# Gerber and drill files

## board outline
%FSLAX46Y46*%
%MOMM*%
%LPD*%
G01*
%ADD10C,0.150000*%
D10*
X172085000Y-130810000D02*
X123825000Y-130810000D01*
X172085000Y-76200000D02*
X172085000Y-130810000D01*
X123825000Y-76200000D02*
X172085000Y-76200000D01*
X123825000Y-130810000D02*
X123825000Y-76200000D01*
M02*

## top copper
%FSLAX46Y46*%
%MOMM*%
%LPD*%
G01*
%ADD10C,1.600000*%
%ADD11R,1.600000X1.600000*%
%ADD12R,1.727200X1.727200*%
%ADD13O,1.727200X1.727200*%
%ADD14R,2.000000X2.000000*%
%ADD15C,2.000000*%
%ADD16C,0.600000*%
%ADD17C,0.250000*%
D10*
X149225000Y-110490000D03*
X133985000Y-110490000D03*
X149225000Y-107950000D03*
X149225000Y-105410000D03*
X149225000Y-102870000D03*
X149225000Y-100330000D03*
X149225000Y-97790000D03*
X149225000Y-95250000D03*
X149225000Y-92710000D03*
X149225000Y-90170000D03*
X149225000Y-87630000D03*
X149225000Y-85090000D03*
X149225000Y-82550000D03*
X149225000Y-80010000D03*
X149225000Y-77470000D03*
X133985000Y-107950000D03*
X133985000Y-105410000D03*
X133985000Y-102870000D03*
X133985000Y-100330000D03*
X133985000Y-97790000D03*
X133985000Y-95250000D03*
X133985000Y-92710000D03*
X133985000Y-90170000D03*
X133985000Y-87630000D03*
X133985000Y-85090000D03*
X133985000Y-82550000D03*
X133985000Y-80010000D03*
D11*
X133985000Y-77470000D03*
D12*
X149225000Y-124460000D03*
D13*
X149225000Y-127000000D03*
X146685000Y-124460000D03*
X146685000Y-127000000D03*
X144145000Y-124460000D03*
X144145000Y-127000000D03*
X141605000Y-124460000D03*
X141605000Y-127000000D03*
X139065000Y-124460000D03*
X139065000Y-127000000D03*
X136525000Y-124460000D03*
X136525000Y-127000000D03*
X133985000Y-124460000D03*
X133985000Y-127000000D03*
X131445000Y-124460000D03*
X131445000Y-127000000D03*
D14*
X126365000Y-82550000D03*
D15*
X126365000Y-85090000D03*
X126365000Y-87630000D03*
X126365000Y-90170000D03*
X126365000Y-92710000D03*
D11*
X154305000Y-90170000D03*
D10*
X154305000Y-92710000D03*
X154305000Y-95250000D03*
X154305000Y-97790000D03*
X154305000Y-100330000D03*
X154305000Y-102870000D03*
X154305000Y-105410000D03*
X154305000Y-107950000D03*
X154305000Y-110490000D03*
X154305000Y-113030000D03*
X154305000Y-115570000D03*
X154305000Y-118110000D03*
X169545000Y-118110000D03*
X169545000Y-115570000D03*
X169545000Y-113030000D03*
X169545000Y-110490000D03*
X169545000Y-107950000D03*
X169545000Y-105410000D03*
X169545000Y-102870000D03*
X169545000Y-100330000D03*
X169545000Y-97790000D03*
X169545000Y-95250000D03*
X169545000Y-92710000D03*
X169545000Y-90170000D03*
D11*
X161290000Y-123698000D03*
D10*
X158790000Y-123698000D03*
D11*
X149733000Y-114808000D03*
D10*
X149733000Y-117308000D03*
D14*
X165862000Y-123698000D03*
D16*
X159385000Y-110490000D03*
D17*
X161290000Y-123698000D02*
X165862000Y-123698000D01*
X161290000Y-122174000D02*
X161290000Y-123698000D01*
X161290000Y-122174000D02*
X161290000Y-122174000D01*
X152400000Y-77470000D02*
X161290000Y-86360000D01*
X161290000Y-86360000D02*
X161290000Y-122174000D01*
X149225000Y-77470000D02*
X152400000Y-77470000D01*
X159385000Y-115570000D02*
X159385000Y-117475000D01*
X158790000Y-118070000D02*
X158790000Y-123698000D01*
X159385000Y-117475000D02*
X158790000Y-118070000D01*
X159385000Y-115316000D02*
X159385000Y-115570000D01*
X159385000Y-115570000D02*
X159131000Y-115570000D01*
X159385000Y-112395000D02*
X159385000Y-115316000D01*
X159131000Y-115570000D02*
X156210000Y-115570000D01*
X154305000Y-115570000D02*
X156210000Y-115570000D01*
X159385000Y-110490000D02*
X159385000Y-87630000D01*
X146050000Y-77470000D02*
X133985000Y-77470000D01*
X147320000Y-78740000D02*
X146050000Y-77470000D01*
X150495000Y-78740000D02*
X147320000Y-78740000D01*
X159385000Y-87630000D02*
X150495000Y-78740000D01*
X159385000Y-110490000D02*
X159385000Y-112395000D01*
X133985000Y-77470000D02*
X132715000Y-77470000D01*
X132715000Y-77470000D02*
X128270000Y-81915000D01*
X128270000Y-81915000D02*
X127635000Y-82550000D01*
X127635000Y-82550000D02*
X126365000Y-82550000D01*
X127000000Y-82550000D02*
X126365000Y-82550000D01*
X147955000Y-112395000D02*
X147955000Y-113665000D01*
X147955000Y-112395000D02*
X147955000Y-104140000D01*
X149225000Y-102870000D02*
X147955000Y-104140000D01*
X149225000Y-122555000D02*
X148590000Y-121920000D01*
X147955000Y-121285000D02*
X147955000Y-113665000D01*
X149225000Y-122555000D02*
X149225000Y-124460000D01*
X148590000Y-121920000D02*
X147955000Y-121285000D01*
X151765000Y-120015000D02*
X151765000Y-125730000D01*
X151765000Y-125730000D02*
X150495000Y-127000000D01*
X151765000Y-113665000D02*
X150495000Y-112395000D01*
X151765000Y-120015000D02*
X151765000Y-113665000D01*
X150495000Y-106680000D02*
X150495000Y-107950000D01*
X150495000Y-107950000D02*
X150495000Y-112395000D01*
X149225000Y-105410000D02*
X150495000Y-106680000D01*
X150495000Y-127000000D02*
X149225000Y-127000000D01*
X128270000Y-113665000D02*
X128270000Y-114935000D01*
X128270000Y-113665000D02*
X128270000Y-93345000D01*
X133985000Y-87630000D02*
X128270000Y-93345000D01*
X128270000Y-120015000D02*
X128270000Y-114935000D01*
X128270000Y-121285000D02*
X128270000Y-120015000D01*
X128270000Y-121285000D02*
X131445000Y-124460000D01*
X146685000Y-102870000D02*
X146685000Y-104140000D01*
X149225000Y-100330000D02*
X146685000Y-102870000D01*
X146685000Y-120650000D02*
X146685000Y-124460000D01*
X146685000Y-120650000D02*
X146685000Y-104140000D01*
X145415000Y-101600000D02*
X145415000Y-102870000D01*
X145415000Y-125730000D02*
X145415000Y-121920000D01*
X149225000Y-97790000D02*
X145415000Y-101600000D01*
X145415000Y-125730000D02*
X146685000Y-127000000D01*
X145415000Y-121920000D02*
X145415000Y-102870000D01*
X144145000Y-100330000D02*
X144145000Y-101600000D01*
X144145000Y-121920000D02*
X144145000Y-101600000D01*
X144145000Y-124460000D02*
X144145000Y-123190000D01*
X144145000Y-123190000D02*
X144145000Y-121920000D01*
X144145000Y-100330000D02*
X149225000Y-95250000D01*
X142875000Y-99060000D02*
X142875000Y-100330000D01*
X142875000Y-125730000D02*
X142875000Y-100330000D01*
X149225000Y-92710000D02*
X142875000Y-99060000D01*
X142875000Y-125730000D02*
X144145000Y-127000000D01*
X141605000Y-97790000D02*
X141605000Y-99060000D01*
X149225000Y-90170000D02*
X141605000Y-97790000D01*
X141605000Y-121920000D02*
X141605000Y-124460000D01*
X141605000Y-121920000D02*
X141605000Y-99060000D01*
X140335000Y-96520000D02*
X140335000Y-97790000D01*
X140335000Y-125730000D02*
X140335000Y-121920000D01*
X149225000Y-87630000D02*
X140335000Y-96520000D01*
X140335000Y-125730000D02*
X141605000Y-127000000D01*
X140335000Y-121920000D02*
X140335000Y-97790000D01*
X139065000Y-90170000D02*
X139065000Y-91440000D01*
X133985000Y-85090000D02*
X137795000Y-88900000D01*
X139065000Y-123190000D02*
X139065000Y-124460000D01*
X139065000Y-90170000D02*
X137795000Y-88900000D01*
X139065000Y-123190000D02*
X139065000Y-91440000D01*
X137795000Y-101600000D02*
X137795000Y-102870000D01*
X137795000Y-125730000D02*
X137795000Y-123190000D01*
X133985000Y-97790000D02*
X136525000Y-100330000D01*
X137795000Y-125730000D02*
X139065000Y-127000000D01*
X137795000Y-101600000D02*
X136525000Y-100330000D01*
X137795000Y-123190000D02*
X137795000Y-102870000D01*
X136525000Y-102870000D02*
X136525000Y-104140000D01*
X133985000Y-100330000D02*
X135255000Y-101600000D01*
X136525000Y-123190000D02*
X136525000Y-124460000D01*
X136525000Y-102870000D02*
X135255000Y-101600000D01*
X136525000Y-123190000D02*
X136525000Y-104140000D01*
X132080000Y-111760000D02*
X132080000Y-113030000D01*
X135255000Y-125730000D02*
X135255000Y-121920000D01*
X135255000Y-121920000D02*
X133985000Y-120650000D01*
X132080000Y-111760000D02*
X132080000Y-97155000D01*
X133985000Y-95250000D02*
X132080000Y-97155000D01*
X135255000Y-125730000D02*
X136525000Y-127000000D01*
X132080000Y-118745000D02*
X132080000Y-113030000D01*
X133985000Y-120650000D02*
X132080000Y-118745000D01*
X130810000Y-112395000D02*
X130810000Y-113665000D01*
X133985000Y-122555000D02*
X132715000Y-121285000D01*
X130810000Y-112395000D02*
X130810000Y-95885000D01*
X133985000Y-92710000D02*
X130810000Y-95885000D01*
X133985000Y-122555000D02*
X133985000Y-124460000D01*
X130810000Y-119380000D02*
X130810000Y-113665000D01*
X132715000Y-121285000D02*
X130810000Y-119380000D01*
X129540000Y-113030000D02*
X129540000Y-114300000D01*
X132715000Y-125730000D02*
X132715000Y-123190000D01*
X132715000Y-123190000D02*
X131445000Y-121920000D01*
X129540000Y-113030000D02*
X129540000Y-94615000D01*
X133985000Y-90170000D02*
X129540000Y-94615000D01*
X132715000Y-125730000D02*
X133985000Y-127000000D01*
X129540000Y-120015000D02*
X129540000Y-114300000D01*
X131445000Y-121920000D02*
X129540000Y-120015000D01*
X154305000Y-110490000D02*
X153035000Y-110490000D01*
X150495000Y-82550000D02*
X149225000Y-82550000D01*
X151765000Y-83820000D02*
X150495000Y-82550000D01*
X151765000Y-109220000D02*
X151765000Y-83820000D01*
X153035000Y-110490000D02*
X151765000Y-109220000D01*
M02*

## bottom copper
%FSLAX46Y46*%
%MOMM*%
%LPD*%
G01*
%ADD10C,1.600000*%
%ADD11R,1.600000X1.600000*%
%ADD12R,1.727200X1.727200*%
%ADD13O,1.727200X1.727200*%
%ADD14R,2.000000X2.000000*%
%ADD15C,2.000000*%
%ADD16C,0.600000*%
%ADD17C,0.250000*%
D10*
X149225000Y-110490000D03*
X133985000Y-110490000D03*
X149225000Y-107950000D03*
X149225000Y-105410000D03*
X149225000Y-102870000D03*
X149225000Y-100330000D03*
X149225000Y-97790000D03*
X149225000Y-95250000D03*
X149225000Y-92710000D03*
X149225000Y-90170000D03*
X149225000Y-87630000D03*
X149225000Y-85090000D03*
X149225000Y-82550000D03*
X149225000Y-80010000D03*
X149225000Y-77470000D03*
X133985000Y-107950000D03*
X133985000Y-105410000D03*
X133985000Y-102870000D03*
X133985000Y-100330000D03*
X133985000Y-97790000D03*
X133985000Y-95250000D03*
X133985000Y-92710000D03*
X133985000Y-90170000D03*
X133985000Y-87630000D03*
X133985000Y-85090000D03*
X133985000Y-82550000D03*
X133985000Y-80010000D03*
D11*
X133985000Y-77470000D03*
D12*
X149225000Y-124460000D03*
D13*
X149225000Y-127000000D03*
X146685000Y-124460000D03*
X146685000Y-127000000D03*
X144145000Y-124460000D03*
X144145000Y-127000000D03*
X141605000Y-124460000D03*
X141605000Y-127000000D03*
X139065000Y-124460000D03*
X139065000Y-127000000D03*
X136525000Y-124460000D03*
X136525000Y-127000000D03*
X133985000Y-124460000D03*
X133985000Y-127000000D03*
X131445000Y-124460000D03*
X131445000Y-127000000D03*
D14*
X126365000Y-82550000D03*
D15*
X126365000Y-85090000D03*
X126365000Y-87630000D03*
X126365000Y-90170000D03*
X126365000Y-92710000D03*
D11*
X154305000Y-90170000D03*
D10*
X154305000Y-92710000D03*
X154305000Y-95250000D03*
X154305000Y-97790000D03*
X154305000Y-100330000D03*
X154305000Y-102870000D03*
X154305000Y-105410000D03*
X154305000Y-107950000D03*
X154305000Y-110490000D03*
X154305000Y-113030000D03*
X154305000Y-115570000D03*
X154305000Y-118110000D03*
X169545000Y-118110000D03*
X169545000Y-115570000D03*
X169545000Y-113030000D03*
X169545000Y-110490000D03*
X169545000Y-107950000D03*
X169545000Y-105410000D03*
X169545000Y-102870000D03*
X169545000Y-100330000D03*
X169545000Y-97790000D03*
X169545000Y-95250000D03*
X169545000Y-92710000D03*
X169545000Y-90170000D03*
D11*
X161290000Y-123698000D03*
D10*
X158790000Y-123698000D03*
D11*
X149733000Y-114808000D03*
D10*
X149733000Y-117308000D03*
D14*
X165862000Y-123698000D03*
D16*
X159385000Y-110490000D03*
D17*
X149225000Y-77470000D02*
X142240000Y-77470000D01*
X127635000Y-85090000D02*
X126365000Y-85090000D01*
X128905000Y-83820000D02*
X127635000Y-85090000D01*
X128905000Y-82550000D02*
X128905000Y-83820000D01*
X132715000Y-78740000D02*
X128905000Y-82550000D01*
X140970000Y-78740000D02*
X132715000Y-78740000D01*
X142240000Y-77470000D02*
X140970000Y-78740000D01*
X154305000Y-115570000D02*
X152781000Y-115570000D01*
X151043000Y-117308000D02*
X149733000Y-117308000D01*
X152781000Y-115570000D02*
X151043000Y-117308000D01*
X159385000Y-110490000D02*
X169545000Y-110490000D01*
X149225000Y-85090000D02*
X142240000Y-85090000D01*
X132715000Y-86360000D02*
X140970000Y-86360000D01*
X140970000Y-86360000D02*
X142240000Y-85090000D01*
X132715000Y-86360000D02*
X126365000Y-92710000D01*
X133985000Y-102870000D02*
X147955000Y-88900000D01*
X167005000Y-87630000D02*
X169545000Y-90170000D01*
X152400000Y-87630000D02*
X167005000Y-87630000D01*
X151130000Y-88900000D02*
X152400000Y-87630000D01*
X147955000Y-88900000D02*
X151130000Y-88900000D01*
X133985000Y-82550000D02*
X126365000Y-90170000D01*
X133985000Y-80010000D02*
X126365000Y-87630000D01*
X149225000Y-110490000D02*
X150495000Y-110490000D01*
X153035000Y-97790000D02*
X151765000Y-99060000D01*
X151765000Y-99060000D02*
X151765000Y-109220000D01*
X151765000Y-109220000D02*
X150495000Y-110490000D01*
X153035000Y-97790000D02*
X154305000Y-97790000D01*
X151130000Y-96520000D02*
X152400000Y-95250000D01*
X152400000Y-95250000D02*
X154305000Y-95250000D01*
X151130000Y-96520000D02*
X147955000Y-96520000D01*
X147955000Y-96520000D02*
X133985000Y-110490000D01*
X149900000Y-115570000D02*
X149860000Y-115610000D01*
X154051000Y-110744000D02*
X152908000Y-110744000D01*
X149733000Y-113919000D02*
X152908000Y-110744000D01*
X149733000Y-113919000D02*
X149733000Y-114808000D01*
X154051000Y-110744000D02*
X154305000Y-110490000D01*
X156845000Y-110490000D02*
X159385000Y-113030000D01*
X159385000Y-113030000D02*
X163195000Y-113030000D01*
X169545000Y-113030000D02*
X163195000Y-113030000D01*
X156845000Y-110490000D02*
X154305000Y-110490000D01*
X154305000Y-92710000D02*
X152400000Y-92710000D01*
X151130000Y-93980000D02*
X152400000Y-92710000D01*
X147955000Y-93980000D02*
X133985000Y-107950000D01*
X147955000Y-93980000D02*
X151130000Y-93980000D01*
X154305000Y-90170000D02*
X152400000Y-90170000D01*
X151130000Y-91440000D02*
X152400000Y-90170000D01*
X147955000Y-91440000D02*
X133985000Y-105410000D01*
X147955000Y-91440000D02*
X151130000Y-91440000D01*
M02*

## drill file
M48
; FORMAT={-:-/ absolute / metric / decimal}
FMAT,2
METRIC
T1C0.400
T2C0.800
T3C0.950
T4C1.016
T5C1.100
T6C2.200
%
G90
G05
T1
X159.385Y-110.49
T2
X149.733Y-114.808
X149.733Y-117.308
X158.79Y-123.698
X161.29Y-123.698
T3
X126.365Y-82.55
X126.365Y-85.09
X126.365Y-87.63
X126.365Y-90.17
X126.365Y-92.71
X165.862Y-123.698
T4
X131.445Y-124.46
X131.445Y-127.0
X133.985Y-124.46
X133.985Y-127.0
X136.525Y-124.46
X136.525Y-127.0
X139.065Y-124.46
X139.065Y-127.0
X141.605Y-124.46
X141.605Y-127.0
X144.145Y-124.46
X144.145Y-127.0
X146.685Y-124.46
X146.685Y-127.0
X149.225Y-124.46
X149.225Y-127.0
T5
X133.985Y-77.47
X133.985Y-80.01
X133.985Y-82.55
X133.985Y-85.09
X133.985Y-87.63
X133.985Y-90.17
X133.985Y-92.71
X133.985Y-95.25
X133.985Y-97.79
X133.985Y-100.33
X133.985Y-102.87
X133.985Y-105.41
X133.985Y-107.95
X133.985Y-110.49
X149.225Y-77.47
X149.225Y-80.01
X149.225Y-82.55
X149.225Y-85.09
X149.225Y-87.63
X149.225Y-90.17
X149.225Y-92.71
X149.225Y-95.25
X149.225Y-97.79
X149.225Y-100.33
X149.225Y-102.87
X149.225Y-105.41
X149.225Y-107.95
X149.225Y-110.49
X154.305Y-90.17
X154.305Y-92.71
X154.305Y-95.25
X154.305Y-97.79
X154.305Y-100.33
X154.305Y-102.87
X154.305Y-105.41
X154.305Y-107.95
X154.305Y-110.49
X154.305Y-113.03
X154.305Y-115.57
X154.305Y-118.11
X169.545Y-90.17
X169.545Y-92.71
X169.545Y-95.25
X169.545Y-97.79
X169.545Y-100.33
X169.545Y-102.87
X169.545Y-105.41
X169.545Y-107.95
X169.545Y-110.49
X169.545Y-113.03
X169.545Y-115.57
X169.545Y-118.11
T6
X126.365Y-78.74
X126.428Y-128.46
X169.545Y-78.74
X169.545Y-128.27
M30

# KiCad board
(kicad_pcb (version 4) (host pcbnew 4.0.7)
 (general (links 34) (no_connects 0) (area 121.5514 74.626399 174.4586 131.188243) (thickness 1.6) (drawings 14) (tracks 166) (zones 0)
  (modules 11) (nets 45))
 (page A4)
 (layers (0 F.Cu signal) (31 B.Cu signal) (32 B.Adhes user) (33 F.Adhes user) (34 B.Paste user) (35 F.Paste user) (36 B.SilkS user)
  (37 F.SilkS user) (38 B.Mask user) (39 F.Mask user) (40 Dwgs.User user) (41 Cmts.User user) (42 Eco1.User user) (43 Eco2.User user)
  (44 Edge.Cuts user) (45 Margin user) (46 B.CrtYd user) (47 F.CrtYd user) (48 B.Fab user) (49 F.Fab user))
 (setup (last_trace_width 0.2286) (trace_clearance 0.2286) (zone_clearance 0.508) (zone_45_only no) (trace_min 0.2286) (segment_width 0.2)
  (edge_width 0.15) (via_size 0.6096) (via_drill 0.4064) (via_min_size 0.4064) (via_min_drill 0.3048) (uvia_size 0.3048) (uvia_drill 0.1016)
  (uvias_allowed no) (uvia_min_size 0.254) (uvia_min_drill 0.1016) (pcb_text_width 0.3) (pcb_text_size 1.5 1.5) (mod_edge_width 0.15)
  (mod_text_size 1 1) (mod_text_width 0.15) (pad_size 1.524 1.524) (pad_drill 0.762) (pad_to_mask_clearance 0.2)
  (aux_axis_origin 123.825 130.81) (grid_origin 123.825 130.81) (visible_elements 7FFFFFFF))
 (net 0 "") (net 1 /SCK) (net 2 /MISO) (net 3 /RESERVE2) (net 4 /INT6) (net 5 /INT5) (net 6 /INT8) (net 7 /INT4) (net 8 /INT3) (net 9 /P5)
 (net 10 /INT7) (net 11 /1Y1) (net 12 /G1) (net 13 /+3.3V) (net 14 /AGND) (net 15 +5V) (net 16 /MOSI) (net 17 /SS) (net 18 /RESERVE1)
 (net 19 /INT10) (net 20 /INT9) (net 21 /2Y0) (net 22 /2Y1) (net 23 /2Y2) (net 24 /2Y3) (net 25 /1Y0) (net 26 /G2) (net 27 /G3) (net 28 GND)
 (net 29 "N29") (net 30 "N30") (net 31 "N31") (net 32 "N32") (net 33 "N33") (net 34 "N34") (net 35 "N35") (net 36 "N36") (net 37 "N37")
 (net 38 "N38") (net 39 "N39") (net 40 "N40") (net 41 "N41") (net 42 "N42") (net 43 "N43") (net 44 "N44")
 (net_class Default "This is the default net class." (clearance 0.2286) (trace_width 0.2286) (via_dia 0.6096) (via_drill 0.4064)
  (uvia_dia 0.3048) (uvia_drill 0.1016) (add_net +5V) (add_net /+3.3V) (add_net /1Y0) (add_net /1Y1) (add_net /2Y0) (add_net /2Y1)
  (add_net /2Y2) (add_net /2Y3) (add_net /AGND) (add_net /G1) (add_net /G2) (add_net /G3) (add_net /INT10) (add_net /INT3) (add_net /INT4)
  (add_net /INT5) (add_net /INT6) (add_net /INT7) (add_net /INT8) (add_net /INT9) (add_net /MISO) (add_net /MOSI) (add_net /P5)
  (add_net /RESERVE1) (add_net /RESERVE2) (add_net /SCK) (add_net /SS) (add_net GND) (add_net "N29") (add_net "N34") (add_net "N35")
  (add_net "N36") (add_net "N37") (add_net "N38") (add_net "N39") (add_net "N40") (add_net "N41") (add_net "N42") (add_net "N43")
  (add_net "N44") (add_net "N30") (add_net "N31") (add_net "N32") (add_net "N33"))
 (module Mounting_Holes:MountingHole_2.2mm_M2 (layer F.Cu) (at 126.4285 128.4605)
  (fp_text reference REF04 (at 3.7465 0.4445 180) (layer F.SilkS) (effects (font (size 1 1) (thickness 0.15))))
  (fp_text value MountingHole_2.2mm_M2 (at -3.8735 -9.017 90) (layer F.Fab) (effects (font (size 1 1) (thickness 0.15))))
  (pad 1 np_thru_hole circle (at 0 0) (size 2.2 2.2) (drill 2.2) (layers *.Cu *.Mask)))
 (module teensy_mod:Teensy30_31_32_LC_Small (layer F.Cu) (at 141.605 93.98 270)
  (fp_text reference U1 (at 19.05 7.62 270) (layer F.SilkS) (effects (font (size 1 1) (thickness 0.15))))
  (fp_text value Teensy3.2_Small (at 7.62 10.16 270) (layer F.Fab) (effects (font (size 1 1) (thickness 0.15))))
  (pad 20 thru_hole circle (at 16.51 -7.62 270) (size 1.6 1.6) (drill 1.1) (layers *.Cu *.Mask F.SilkS) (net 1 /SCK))
  (pad 14 thru_hole circle (at 16.51 7.62 270) (size 1.6 1.6) (drill 1.1) (layers *.Cu *.Mask F.SilkS) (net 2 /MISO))
  (pad 21 thru_hole circle (at 13.97 -7.62 270) (size 1.6 1.6) (drill 1.1) (layers *.Cu *.Mask F.SilkS) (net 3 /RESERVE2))
  (pad 22 thru_hole circle (at 11.43 -7.62 270) (size 1.6 1.6) (drill 1.1) (layers *.Cu *.Mask F.SilkS) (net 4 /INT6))
  (pad 23 thru_hole circle (at 8.89 -7.62 270) (size 1.6 1.6) (drill 1.1) (layers *.Cu *.Mask F.SilkS) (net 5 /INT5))
  (pad 24 thru_hole circle (at 6.35 -7.62 270) (size 1.6 1.6) (drill 1.1) (layers *.Cu *.Mask F.SilkS) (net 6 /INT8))
  (pad 25 thru_hole circle (at 3.81 -7.62 270) (size 1.6 1.6) (drill 1.1) (layers *.Cu *.Mask F.SilkS) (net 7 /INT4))
  (pad 26 thru_hole circle (at 1.27 -7.62 270) (size 1.6 1.6) (drill 1.1) (layers *.Cu *.Mask F.SilkS) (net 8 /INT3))
  (pad 27 thru_hole circle (at -1.27 -7.62 270) (size 1.6 1.6) (drill 1.1) (layers *.Cu *.Mask F.SilkS) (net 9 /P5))
  (pad 28 thru_hole circle (at -3.81 -7.62 270) (size 1.6 1.6) (drill 1.1) (layers *.Cu *.Mask F.SilkS) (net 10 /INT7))
  (pad 29 thru_hole circle (at -6.35 -7.62 270) (size 1.6 1.6) (drill 1.1) (layers *.Cu *.Mask F.SilkS) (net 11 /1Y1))
  (pad 30 thru_hole circle (at -8.89 -7.62 270) (size 1.6 1.6) (drill 1.1) (layers *.Cu *.Mask F.SilkS) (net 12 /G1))
  (pad 31 thru_hole circle (at -11.43 -7.62 270) (size 1.6 1.6) (drill 1.1) (layers *.Cu *.Mask F.SilkS) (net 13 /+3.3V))
  (pad 32 thru_hole circle (at -13.97 -7.62 270) (size 1.6 1.6) (drill 1.1) (layers *.Cu *.Mask F.SilkS) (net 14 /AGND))
  (pad 33 thru_hole circle (at -16.51 -7.62 270) (size 1.6 1.6) (drill 1.1) (layers *.Cu *.Mask F.SilkS) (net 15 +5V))
  (pad 13 thru_hole circle (at 13.97 7.62 270) (size 1.6 1.6) (drill 1.1) (layers *.Cu *.Mask F.SilkS) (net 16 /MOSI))
  (pad 12 thru_hole circle (at 11.43 7.62 270) (size 1.6 1.6) (drill 1.1) (layers *.Cu *.Mask F.SilkS) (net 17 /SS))
  (pad 11 thru_hole circle (at 8.89 7.62 270) (size 1.6 1.6) (drill 1.1) (layers *.Cu *.Mask F.SilkS) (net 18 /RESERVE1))
  (pad 10 thru_hole circle (at 6.35 7.62 270) (size 1.6 1.6) (drill 1.1) (layers *.Cu *.Mask F.SilkS) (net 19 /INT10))
  (pad 9 thru_hole circle (at 3.81 7.62 270) (size 1.6 1.6) (drill 1.1) (layers *.Cu *.Mask F.SilkS) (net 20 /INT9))
  (pad 8 thru_hole circle (at 1.27 7.62 270) (size 1.6 1.6) (drill 1.1) (layers *.Cu *.Mask F.SilkS) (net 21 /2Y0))
  (pad 7 thru_hole circle (at -1.27 7.62 270) (size 1.6 1.6) (drill 1.1) (layers *.Cu *.Mask F.SilkS) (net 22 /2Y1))
  (pad 6 thru_hole circle (at -3.81 7.62 270) (size 1.6 1.6) (drill 1.1) (layers *.Cu *.Mask F.SilkS) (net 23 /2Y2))
  (pad 5 thru_hole circle (at -6.35 7.62 270) (size 1.6 1.6) (drill 1.1) (layers *.Cu *.Mask F.SilkS) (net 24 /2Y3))
  (pad 4 thru_hole circle (at -8.89 7.62 270) (size 1.6 1.6) (drill 1.1) (layers *.Cu *.Mask F.SilkS) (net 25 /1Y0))
  (pad 3 thru_hole circle (at -11.43 7.62 270) (size 1.6 1.6) (drill 1.1) (layers *.Cu *.Mask F.SilkS) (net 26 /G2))
  (pad 2 thru_hole circle (at -13.97 7.62 270) (size 1.6 1.6) (drill 1.1) (layers *.Cu *.Mask F.SilkS) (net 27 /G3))
  (pad 1 thru_hole rect (at -16.51 7.62 270) (size 1.6 1.6) (drill 1.1) (layers *.Cu *.Mask F.SilkS) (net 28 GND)))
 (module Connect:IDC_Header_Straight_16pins (layer F.Cu) (at 149.225 124.46 180)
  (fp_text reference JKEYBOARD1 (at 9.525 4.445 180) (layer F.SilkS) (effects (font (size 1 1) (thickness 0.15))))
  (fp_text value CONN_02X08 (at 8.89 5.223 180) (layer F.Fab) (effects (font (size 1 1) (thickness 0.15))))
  (pad 1 thru_hole rect (at 0 0 180) (size 1.7272 1.7272) (drill 1.016) (layers *.Cu *.Mask) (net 5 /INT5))
  (pad 2 thru_hole oval (at 0 -2.54 180) (size 1.7272 1.7272) (drill 1.016) (layers *.Cu *.Mask) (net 4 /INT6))
  (pad 3 thru_hole oval (at 2.54 0 180) (size 1.7272 1.7272) (drill 1.016) (layers *.Cu *.Mask) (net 6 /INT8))
  (pad 4 thru_hole oval (at 2.54 -2.54 180) (size 1.7272 1.7272) (drill 1.016) (layers *.Cu *.Mask) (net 7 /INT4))
  (pad 5 thru_hole oval (at 5.08 0 180) (size 1.7272 1.7272) (drill 1.016) (layers *.Cu *.Mask) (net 8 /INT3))
  (pad 6 thru_hole oval (at 5.08 -2.54 180) (size 1.7272 1.7272) (drill 1.016) (layers *.Cu *.Mask) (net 9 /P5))
  (pad 7 thru_hole oval (at 7.62 0 180) (size 1.7272 1.7272) (drill 1.016) (layers *.Cu *.Mask) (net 10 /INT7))
  (pad 8 thru_hole oval (at 7.62 -2.54 180) (size 1.7272 1.7272) (drill 1.016) (layers *.Cu *.Mask) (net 11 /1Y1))
  (pad 9 thru_hole oval (at 10.16 0 180) (size 1.7272 1.7272) (drill 1.016) (layers *.Cu *.Mask) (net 25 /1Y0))
  (pad 10 thru_hole oval (at 10.16 -2.54 180) (size 1.7272 1.7272) (drill 1.016) (layers *.Cu *.Mask) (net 20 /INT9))
  (pad 11 thru_hole oval (at 12.7 0 180) (size 1.7272 1.7272) (drill 1.016) (layers *.Cu *.Mask) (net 19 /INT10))
  (pad 12 thru_hole oval (at 12.7 -2.54 180) (size 1.7272 1.7272) (drill 1.016) (layers *.Cu *.Mask) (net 21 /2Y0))
  (pad 13 thru_hole oval (at 15.24 0 180) (size 1.7272 1.7272) (drill 1.016) (layers *.Cu *.Mask) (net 22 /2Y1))
  (pad 14 thru_hole oval (at 15.24 -2.54 180) (size 1.7272 1.7272) (drill 1.016) (layers *.Cu *.Mask) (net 23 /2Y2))
  (pad 15 thru_hole oval (at 17.78 0 180) (size 1.7272 1.7272) (drill 1.016) (layers *.Cu *.Mask) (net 24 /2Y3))
  (pad 16 thru_hole oval (at 17.78 -2.54 180) (size 1.7272 1.7272) (drill 1.016) (layers *.Cu *.Mask) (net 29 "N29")))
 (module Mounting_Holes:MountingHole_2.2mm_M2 (layer F.Cu) (at 169.545 128.27)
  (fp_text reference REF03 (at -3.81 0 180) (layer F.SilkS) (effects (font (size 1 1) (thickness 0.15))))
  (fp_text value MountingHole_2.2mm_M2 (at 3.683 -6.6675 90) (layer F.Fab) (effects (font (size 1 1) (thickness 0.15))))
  (pad 1 np_thru_hole circle (at 0 0) (size 2.2 2.2) (drill 2.2) (layers *.Cu *.Mask)))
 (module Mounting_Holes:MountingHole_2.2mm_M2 (layer F.Cu) (at 169.545 78.74)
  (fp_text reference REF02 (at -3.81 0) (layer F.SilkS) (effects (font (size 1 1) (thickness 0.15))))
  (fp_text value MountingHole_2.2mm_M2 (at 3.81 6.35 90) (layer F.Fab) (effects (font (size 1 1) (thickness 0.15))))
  (pad 1 np_thru_hole circle (at 0 0) (size 2.2 2.2) (drill 2.2) (layers *.Cu *.Mask)))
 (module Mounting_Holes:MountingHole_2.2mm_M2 (layer F.Cu) (at 126.365 78.74)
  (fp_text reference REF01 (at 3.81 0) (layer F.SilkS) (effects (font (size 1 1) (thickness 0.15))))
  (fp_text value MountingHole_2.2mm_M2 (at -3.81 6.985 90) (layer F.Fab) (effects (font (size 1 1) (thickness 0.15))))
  (pad 1 np_thru_hole circle (at 0 0) (size 2.2 2.2) (drill 2.2) (layers *.Cu *.Mask)))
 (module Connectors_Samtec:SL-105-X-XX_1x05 (layer F.Cu) (at 126.365 82.55)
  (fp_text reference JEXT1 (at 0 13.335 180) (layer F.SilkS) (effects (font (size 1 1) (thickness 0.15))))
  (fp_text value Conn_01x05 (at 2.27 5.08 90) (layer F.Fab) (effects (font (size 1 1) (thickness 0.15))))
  (pad 1 thru_hole rect (at 0 0) (size 2 2) (drill 0.95) (layers *.Cu *.Mask) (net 28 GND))
  (pad 2 thru_hole circle (at 0 2.54) (size 2 2) (drill 0.95) (layers *.Cu *.Mask) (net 15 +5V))
  (pad 3 thru_hole circle (at 0 5.08) (size 2 2) (drill 0.95) (layers *.Cu *.Mask) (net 27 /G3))
  (pad 4 thru_hole circle (at 0 7.62) (size 2 2) (drill 0.95) (layers *.Cu *.Mask) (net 26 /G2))
  (pad 5 thru_hole circle (at 0 10.16) (size 2 2) (drill 0.95) (layers *.Cu *.Mask) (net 12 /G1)))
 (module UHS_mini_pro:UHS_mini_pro (layer F.Cu) (at 161.925 104.14 270)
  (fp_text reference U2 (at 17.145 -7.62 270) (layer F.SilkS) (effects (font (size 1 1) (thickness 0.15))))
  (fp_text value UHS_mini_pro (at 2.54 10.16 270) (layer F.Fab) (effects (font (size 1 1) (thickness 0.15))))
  (pad 1 thru_hole rect (at -13.97 7.62 270) (size 1.6 1.6) (drill 1.1) (layers *.Cu *.Mask F.SilkS) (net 17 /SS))
  (pad 2 thru_hole circle (at -11.43 7.62 270) (size 1.6 1.6) (drill 1.1) (layers *.Cu *.Mask F.SilkS) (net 16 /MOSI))
  (pad 3 thru_hole circle (at -8.89 7.62 270) (size 1.6 1.6) (drill 1.1) (layers *.Cu *.Mask F.SilkS) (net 2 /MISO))
  (pad 4 thru_hole circle (at -6.35 7.62 270) (size 1.6 1.6) (drill 1.1) (layers *.Cu *.Mask F.SilkS) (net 1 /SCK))
  (pad 5 thru_hole circle (at -3.81 7.62 270) (size 1.6 1.6) (drill 1.1) (layers *.Cu *.Mask F.SilkS) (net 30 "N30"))
  (pad 6 thru_hole circle (at -1.27 7.62 270) (size 1.6 1.6) (drill 1.1) (layers *.Cu *.Mask F.SilkS) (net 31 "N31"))
  (pad 7 thru_hole circle (at 1.27 7.62 270) (size 1.6 1.6) (drill 1.1) (layers *.Cu *.Mask F.SilkS) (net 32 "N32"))
  (pad 8 thru_hole circle (at 3.81 7.62 270) (size 1.6 1.6) (drill 1.1) (layers *.Cu *.Mask F.SilkS) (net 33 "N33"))
  (pad 9 thru_hole circle (at 6.35 7.62 270) (size 1.6 1.6) (drill 1.1) (layers *.Cu *.Mask F.SilkS) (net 13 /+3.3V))
  (pad 10 thru_hole circle (at 8.89 7.62 270) (size 1.6 1.6) (drill 1.1) (layers *.Cu *.Mask F.SilkS) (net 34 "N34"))
  (pad 11 thru_hole circle (at 11.43 7.62 270) (size 1.6 1.6) (drill 1.1) (layers *.Cu *.Mask F.SilkS) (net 28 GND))
  (pad 12 thru_hole circle (at 13.97 7.62 270) (size 1.6 1.6) (drill 1.1) (layers *.Cu *.Mask F.SilkS) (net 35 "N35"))
  (pad 13 thru_hole circle (at 13.97 -7.62 270) (size 1.6 1.6) (drill 1.1) (layers *.Cu *.Mask F.SilkS) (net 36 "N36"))
  (pad 14 thru_hole circle (at 11.43 -7.62 270) (size 1.6 1.6) (drill 1.1) (layers *.Cu *.Mask F.SilkS) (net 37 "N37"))
  (pad 15 thru_hole circle (at 8.89 -7.62 270) (size 1.6 1.6) (drill 1.1) (layers *.Cu *.Mask F.SilkS) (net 13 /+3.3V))
  (pad 16 thru_hole circle (at 6.35 -7.62 270) (size 1.6 1.6) (drill 1.1) (layers *.Cu *.Mask F.SilkS) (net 28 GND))
  (pad 17 thru_hole circle (at 3.81 -7.62 270) (size 1.6 1.6) (drill 1.1) (layers *.Cu *.Mask F.SilkS) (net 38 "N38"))
  (pad 18 thru_hole circle (at 1.27 -7.62 270) (size 1.6 1.6) (drill 1.1) (layers *.Cu *.Mask F.SilkS) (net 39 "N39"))
  (pad 19 thru_hole circle (at -1.27 -7.62 270) (size 1.6 1.6) (drill 1.1) (layers *.Cu *.Mask F.SilkS) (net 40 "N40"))
  (pad 20 thru_hole circle (at -3.81 -7.62 270) (size 1.6 1.6) (drill 1.1) (layers *.Cu *.Mask F.SilkS) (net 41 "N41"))
  (pad 21 thru_hole circle (at -6.35 -7.62 270) (size 1.6 1.6) (drill 1.1) (layers *.Cu *.Mask F.SilkS) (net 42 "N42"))
  (pad 22 thru_hole circle (at -8.89 -7.62 270) (size 1.6 1.6) (drill 1.1) (layers *.Cu *.Mask F.SilkS) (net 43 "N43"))
  (pad 23 thru_hole circle (at -11.43 -7.62 270) (size 1.6 1.6) (drill 1.1) (layers *.Cu *.Mask F.SilkS) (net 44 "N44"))
  (pad 24 thru_hole circle (at -13.97 -7.62 270) (size 1.6 1.6) (drill 1.1) (layers *.Cu *.Mask F.SilkS) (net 18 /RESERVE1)))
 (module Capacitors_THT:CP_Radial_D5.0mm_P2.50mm (layer F.Cu) (at 161.29 123.698 180)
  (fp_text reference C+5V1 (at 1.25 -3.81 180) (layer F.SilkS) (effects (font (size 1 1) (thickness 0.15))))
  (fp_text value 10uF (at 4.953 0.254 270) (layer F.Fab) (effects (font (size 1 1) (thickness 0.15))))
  (pad 1 thru_hole rect (at 0 0 180) (size 1.6 1.6) (drill 0.8) (layers *.Cu *.Mask) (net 15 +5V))
  (pad 2 thru_hole circle (at 2.5 0 180) (size 1.6 1.6) (drill 0.8) (layers *.Cu *.Mask) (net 28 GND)))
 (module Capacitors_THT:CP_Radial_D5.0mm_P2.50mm (layer F.Cu) (at 149.733 114.808 270)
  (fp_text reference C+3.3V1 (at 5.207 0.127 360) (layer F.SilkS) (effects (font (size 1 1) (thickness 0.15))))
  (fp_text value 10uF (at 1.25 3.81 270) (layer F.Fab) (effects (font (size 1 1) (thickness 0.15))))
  (pad 1 thru_hole rect (at 0 0 270) (size 1.6 1.6) (drill 0.8) (layers *.Cu *.Mask) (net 13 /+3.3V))
  (pad 2 thru_hole circle (at 2.5 0 270) (size 1.6 1.6) (drill 0.8) (layers *.Cu *.Mask) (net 28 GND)))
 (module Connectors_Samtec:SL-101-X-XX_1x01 (layer F.Cu) (at 165.862 123.698)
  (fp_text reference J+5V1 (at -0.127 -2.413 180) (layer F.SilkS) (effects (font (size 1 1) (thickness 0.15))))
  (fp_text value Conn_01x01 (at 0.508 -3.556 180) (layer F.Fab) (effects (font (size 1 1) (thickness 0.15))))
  (pad 1 thru_hole rect (at 0 0) (size 2 2) (drill 0.95) (layers *.Cu *.Mask) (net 15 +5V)))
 (gr_line (start 172.085 130.81) (end 123.825 130.81) (angle 90) (layer Edge.Cuts) (width 0.15))
 (gr_line (start 172.085 76.2) (end 172.085 130.81) (angle 90) (layer Edge.Cuts) (width 0.15))
 (gr_line (start 123.825 76.2) (end 172.085 76.2) (angle 90) (layer Edge.Cuts) (width 0.15))
 (gr_line (start 123.825 130.81) (end 123.825 76.2) (angle 90) (layer Edge.Cuts) (width 0.15))
 (segment (start 161.29 123.698) (end 165.862 123.698) (width 0.25) (layer F.Cu) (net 15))
 (segment (start 161.29 122.174) (end 161.29 123.698) (width 0.25) (layer F.Cu) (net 15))
 (segment (start 161.29 122.174) (end 161.29 122.174) (width 0.25) (layer F.Cu) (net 15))
 (segment (start 152.4 77.47) (end 161.29 86.36) (width 0.25) (layer F.Cu) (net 15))
 (segment (start 161.29 86.36) (end 161.29 122.174) (width 0.25) (layer F.Cu) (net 15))
 (segment (start 149.225 77.47) (end 152.4 77.47) (width 0.25) (layer F.Cu) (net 15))
 (segment (start 149.225 77.47) (end 142.24 77.47) (width 0.25) (layer B.Cu) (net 15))
 (segment (start 127.635 85.09) (end 126.365 85.09) (width 0.25) (layer B.Cu) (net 15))
 (segment (start 128.905 83.82) (end 127.635 85.09) (width 0.25) (layer B.Cu) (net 15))
 (segment (start 128.905 82.55) (end 128.905 83.82) (width 0.25) (layer B.Cu) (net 15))
 (segment (start 132.715 78.74) (end 128.905 82.55) (width 0.25) (layer B.Cu) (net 15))
 (segment (start 140.97 78.74) (end 132.715 78.74) (width 0.25) (layer B.Cu) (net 15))
 (segment (start 142.24 77.47) (end 140.97 78.74) (width 0.25) (layer B.Cu) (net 15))
 (segment (start 159.385 115.57) (end 159.385 117.475) (width 0.25) (layer F.Cu) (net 28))
 (segment (start 158.79 118.07) (end 158.79 123.698) (width 0.25) (layer F.Cu) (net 28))
 (segment (start 159.385 117.475) (end 158.79 118.07) (width 0.25) (layer F.Cu) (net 28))
 (segment (start 159.385 115.316) (end 159.385 115.57) (width 0.25) (layer F.Cu) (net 28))
 (segment (start 159.385 115.57) (end 159.131 115.57) (width 0.25) (layer F.Cu) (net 28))
 (segment (start 159.385 112.395) (end 159.385 115.316) (width 0.25) (layer F.Cu) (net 28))
 (segment (start 159.131 115.57) (end 156.21 115.57) (width 0.25) (layer F.Cu) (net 28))
 (segment (start 154.305 115.57) (end 156.21 115.57) (width 0.25) (layer F.Cu) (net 28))
 (segment (start 154.305 115.57) (end 152.781 115.57) (width 0.25) (layer B.Cu) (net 28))
 (segment (start 151.043 117.308) (end 149.733 117.308) (width 0.25) (layer B.Cu) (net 28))
 (segment (start 152.781 115.57) (end 151.043 117.308) (width 0.25) (layer B.Cu) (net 28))
 (segment (start 159.385 110.49) (end 159.385 87.63) (width 0.25) (layer F.Cu) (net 28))
 (segment (start 146.05 77.47) (end 133.985 77.47) (width 0.25) (layer F.Cu) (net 28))
 (segment (start 147.32 78.74) (end 146.05 77.47) (width 0.25) (layer F.Cu) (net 28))
 (segment (start 150.495 78.74) (end 147.32 78.74) (width 0.25) (layer F.Cu) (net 28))
 (segment (start 159.385 87.63) (end 150.495 78.74) (width 0.25) (layer F.Cu) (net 28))
 (via (at 159.385 110.49) (size 0.6) (drill 0.4) (layers F.Cu B.Cu) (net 28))
 (segment (start 159.385 110.49) (end 159.385 112.395) (width 0.25) (layer F.Cu) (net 28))
 (segment (start 159.385 110.49) (end 169.545 110.49) (width 0.25) (layer B.Cu) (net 28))
 (segment (start 133.985 77.47) (end 132.715 77.47) (width 0.25) (layer F.Cu) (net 28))
 (segment (start 132.715 77.47) (end 128.27 81.915) (width 0.25) (layer F.Cu) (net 28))
 (segment (start 128.27 81.915) (end 127.635 82.55) (width 0.25) (layer F.Cu) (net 28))
 (segment (start 127.635 82.55) (end 126.365 82.55) (width 0.25) (layer F.Cu) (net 28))
 (segment (start 127 82.55) (end 126.365 82.55) (width 0.25) (layer F.Cu) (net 28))
 (segment (start 147.955 112.395) (end 147.955 113.665) (width 0.25) (layer F.Cu) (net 5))
 (segment (start 147.955 112.395) (end 147.955 104.14) (width 0.25) (layer F.Cu) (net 5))
 (segment (start 149.225 102.87) (end 147.955 104.14) (width 0.25) (layer F.Cu) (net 5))
 (segment (start 149.225 122.555) (end 148.59 121.92) (width 0.25) (layer F.Cu) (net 5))
 (segment (start 147.955 121.285) (end 147.955 113.665) (width 0.25) (layer F.Cu) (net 5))
 (segment (start 149.225 122.555) (end 149.225 124.46) (width 0.25) (layer F.Cu) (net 5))
 (segment (start 148.59 121.92) (end 147.955 121.285) (width 0.25) (layer F.Cu) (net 5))
 (segment (start 151.765 120.015) (end 151.765 125.73) (width 0.25) (layer F.Cu) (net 4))
 (segment (start 151.765 125.73) (end 150.495 127) (width 0.25) (layer F.Cu) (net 4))
 (segment (start 151.765 113.665) (end 150.495 112.395) (width 0.25) (layer F.Cu) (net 4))
 (segment (start 151.765 120.015) (end 151.765 113.665) (width 0.25) (layer F.Cu) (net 4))
 (segment (start 150.495 106.68) (end 150.495 107.95) (width 0.25) (layer F.Cu) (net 4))
 (segment (start 150.495 107.95) (end 150.495 112.395) (width 0.25) (layer F.Cu) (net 4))
 (segment (start 149.225 105.41) (end 150.495 106.68) (width 0.25) (layer F.Cu) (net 4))
 (segment (start 150.495 127) (end 149.225 127) (width 0.25) (layer F.Cu) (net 4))
 (segment (start 128.27 113.665) (end 128.27 114.935) (width 0.25) (layer F.Cu) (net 24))
 (segment (start 128.27 113.665) (end 128.27 93.345) (width 0.25) (layer F.Cu) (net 24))
 (segment (start 133.985 87.63) (end 128.27 93.345) (width 0.25) (layer F.Cu) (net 24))
 (segment (start 128.27 120.015) (end 128.27 114.935) (width 0.25) (layer F.Cu) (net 24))
 (segment (start 128.27 121.285) (end 128.27 120.015) (width 0.25) (layer F.Cu) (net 24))
 (segment (start 128.27 121.285) (end 131.445 124.46) (width 0.25) (layer F.Cu) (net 24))
 (segment (start 149.225 85.09) (end 142.24 85.09) (width 0.25) (layer B.Cu) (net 12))
 (segment (start 132.715 86.36) (end 140.97 86.36) (width 0.25) (layer B.Cu) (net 12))
 (segment (start 140.97 86.36) (end 142.24 85.09) (width 0.25) (layer B.Cu) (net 12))
 (segment (start 132.715 86.36) (end 126.365 92.71) (width 0.25) (layer B.Cu) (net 12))
 (segment (start 133.985 102.87) (end 147.955 88.9) (width 0.25) (layer B.Cu) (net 18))
 (segment (start 167.005 87.63) (end 169.545 90.17) (width 0.25) (layer B.Cu) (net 18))
 (segment (start 152.4 87.63) (end 167.005 87.63) (width 0.25) (layer B.Cu) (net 18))
 (segment (start 151.13 88.9) (end 152.4 87.63) (width 0.25) (layer B.Cu) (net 18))
 (segment (start 147.955 88.9) (end 151.13 88.9) (width 0.25) (layer B.Cu) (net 18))
 (segment (start 133.985 82.55) (end 126.365 90.17) (width 0.25) (layer B.Cu) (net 26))
 (segment (start 133.985 80.01) (end 126.365 87.63) (width 0.25) (layer B.Cu) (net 27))
 (segment (start 146.685 102.87) (end 146.685 104.14) (width 0.25) (layer F.Cu) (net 6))
 (segment (start 149.225 100.33) (end 146.685 102.87) (width 0.25) (layer F.Cu) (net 6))
 (segment (start 146.685 120.65) (end 146.685 124.46) (width 0.25) (layer F.Cu) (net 6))
 (segment (start 146.685 120.65) (end 146.685 104.14) (width 0.25) (layer F.Cu) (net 6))
 (segment (start 145.415 101.6) (end 145.415 102.87) (width 0.25) (layer F.Cu) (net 7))
 (segment (start 145.415 125.73) (end 145.415 121.92) (width 0.25) (layer F.Cu) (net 7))
 (segment (start 149.225 97.79) (end 145.415 101.6) (width 0.25) (layer F.Cu) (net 7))
 (segment (start 145.415 125.73) (end 146.685 127) (width 0.25) (layer F.Cu) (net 7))
 (segment (start 145.415 121.92) (end 145.415 102.87) (width 0.25) (layer F.Cu) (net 7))
 (segment (start 144.145 100.33) (end 144.145 101.6) (width 0.25) (layer F.Cu) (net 8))
 (segment (start 144.145 121.92) (end 144.145 101.6) (width 0.25) (layer F.Cu) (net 8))
 (segment (start 144.145 124.46) (end 144.145 123.19) (width 0.25) (layer F.Cu) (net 8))
 (segment (start 144.145 123.19) (end 144.145 121.92) (width 0.25) (layer F.Cu) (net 8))
 (segment (start 144.145 100.33) (end 149.225 95.25) (width 0.25) (layer F.Cu) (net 8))
 (segment (start 142.875 99.06) (end 142.875 100.33) (width 0.25) (layer F.Cu) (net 9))
 (segment (start 142.875 125.73) (end 142.875 100.33) (width 0.25) (layer F.Cu) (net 9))
 (segment (start 149.225 92.71) (end 142.875 99.06) (width 0.25) (layer F.Cu) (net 9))
 (segment (start 142.875 125.73) (end 144.145 127) (width 0.25) (layer F.Cu) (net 9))
 (segment (start 141.605 97.79) (end 141.605 99.06) (width 0.25) (layer F.Cu) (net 10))
 (segment (start 149.225 90.17) (end 141.605 97.79) (width 0.25) (layer F.Cu) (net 10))
 (segment (start 141.605 121.92) (end 141.605 124.46) (width 0.25) (layer F.Cu) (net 10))
 (segment (start 141.605 121.92) (end 141.605 99.06) (width 0.25) (layer F.Cu) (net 10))
 (segment (start 140.335 96.52) (end 140.335 97.79) (width 0.25) (layer F.Cu) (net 11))
 (segment (start 140.335 125.73) (end 140.335 121.92) (width 0.25) (layer F.Cu) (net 11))
 (segment (start 149.225 87.63) (end 140.335 96.52) (width 0.25) (layer F.Cu) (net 11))
 (segment (start 140.335 125.73) (end 141.605 127) (width 0.25) (layer F.Cu) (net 11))
 (segment (start 140.335 121.92) (end 140.335 97.79) (width 0.25) (layer F.Cu) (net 11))
 (segment (start 139.065 90.17) (end 139.065 91.44) (width 0.25) (layer F.Cu) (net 25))
 (segment (start 133.985 85.09) (end 137.795 88.9) (width 0.25) (layer F.Cu) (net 25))
 (segment (start 139.065 123.19) (end 139.065 124.46) (width 0.25) (layer F.Cu) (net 25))
 (segment (start 139.065 90.17) (end 137.795 88.9) (width 0.25) (layer F.Cu) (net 25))
 (segment (start 139.065 123.19) (end 139.065 91.44) (width 0.25) (layer F.Cu) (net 25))
 (segment (start 137.795 101.6) (end 137.795 102.87) (width 0.25) (layer F.Cu) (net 20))
 (segment (start 137.795 125.73) (end 137.795 123.19) (width 0.25) (layer F.Cu) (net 20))
 (segment (start 133.985 97.79) (end 136.525 100.33) (width 0.25) (layer F.Cu) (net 20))
 (segment (start 137.795 125.73) (end 139.065 127) (width 0.25) (layer F.Cu) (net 20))
 (segment (start 137.795 101.6) (end 136.525 100.33) (width 0.25) (layer F.Cu) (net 20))
 (segment (start 137.795 123.19) (end 137.795 102.87) (width 0.25) (layer F.Cu) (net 20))
 (segment (start 136.525 102.87) (end 136.525 104.14) (width 0.25) (layer F.Cu) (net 19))
 (segment (start 133.985 100.33) (end 135.255 101.6) (width 0.25) (layer F.Cu) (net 19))
 (segment (start 136.525 123.19) (end 136.525 124.46) (width 0.25) (layer F.Cu) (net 19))
 (segment (start 136.525 102.87) (end 135.255 101.6) (width 0.25) (layer F.Cu) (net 19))
 (segment (start 136.525 123.19) (end 136.525 104.14) (width 0.25) (layer F.Cu) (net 19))
 (segment (start 132.08 111.76) (end 132.08 113.03) (width 0.25) (layer F.Cu) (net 21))
 (segment (start 135.255 125.73) (end 135.255 121.92) (width 0.25) (layer F.Cu) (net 21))
 (segment (start 135.255 121.92) (end 133.985 120.65) (width 0.25) (layer F.Cu) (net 21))
 (segment (start 132.08 111.76) (end 132.08 97.155) (width 0.25) (layer F.Cu) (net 21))
 (segment (start 133.985 95.25) (end 132.08 97.155) (width 0.25) (layer F.Cu) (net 21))
 (segment (start 135.255 125.73) (end 136.525 127) (width 0.25) (layer F.Cu) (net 21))
 (segment (start 132.08 118.745) (end 132.08 113.03) (width 0.25) (layer F.Cu) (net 21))
 (segment (start 133.985 120.65) (end 132.08 118.745) (width 0.25) (layer F.Cu) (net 21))
 (segment (start 130.81 112.395) (end 130.81 113.665) (width 0.25) (layer F.Cu) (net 22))
 (segment (start 133.985 122.555) (end 132.715 121.285) (width 0.25) (layer F.Cu) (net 22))
 (segment (start 130.81 112.395) (end 130.81 95.885) (width 0.25) (layer F.Cu) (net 22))
 (segment (start 133.985 92.71) (end 130.81 95.885) (width 0.25) (layer F.Cu) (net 22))
 (segment (start 133.985 122.555) (end 133.985 124.46) (width 0.25) (layer F.Cu) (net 22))
 (segment (start 130.81 119.38) (end 130.81 113.665) (width 0.25) (layer F.Cu) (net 22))
 (segment (start 132.715 121.285) (end 130.81 119.38) (width 0.25) (layer F.Cu) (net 22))
 (segment (start 129.54 113.03) (end 129.54 114.3) (width 0.25) (layer F.Cu) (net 23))
 (segment (start 132.715 125.73) (end 132.715 123.19) (width 0.25) (layer F.Cu) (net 23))
 (segment (start 132.715 123.19) (end 131.445 121.92) (width 0.25) (layer F.Cu) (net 23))
 (segment (start 129.54 113.03) (end 129.54 94.615) (width 0.25) (layer F.Cu) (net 23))
 (segment (start 133.985 90.17) (end 129.54 94.615) (width 0.25) (layer F.Cu) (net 23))
 (segment (start 132.715 125.73) (end 133.985 127) (width 0.25) (layer F.Cu) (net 23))
 (segment (start 129.54 120.015) (end 129.54 114.3) (width 0.25) (layer F.Cu) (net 23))
 (segment (start 131.445 121.92) (end 129.54 120.015) (width 0.25) (layer F.Cu) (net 23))
 (segment (start 149.225 110.49) (end 150.495 110.49) (width 0.25) (layer B.Cu) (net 1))
 (segment (start 153.035 97.79) (end 151.765 99.06) (width 0.25) (layer B.Cu) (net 1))
 (segment (start 151.765 99.06) (end 151.765 109.22) (width 0.25) (layer B.Cu) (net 1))
 (segment (start 151.765 109.22) (end 150.495 110.49) (width 0.25) (layer B.Cu) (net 1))
 (segment (start 153.035 97.79) (end 154.305 97.79) (width 0.25) (layer B.Cu) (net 1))
 (segment (start 151.13 96.52) (end 152.4 95.25) (width 0.25) (layer B.Cu) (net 2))
 (segment (start 152.4 95.25) (end 154.305 95.25) (width 0.25) (layer B.Cu) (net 2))
 (segment (start 151.13 96.52) (end 147.955 96.52) (width 0.25) (layer B.Cu) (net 2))
 (segment (start 147.955 96.52) (end 133.985 110.49) (width 0.25) (layer B.Cu) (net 2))
 (segment (start 149.9 115.57) (end 149.86 115.61) (width 0.25) (layer B.Cu) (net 13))
 (segment (start 154.051 110.744) (end 152.908 110.744) (width 0.25) (layer B.Cu) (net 13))
 (segment (start 149.733 113.919) (end 152.908 110.744) (width 0.25) (layer B.Cu) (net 13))
 (segment (start 149.733 113.919) (end 149.733 114.808) (width 0.25) (layer B.Cu) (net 13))
 (segment (start 154.051 110.744) (end 154.305 110.49) (width 0.25) (layer B.Cu) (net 13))
 (segment (start 156.845 110.49) (end 159.385 113.03) (width 0.25) (layer B.Cu) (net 13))
 (segment (start 159.385 113.03) (end 163.195 113.03) (width 0.25) (layer B.Cu) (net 13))
 (segment (start 169.545 113.03) (end 163.195 113.03) (width 0.25) (layer B.Cu) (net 13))
 (segment (start 156.845 110.49) (end 154.305 110.49) (width 0.25) (layer B.Cu) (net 13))
 (segment (start 154.305 110.49) (end 153.035 110.49) (width 0.25) (layer F.Cu) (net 13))
 (segment (start 150.495 82.55) (end 149.225 82.55) (width 0.25) (layer F.Cu) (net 13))
 (segment (start 151.765 83.82) (end 150.495 82.55) (width 0.25) (layer F.Cu) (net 13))
 (segment (start 151.765 109.22) (end 151.765 83.82) (width 0.25) (layer F.Cu) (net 13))
 (segment (start 153.035 110.49) (end 151.765 109.22) (width 0.25) (layer F.Cu) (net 13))
 (segment (start 154.305 92.71) (end 152.4 92.71) (width 0.25) (layer B.Cu) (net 16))
 (segment (start 151.13 93.98) (end 152.4 92.71) (width 0.25) (layer B.Cu) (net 16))
 (segment (start 147.955 93.98) (end 133.985 107.95) (width 0.25) (layer B.Cu) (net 16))
 (segment (start 147.955 93.98) (end 151.13 93.98) (width 0.25) (layer B.Cu) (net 16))
 (segment (start 154.305 90.17) (end 152.4 90.17) (width 0.25) (layer B.Cu) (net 17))
 (segment (start 151.13 91.44) (end 152.4 90.17) (width 0.25) (layer B.Cu) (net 17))
 (segment (start 147.955 91.44) (end 133.985 105.41) (width 0.25) (layer B.Cu) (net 17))
 (segment (start 147.955 91.44) (end 151.13 91.44) (width 0.25) (layer B.Cu) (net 17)))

